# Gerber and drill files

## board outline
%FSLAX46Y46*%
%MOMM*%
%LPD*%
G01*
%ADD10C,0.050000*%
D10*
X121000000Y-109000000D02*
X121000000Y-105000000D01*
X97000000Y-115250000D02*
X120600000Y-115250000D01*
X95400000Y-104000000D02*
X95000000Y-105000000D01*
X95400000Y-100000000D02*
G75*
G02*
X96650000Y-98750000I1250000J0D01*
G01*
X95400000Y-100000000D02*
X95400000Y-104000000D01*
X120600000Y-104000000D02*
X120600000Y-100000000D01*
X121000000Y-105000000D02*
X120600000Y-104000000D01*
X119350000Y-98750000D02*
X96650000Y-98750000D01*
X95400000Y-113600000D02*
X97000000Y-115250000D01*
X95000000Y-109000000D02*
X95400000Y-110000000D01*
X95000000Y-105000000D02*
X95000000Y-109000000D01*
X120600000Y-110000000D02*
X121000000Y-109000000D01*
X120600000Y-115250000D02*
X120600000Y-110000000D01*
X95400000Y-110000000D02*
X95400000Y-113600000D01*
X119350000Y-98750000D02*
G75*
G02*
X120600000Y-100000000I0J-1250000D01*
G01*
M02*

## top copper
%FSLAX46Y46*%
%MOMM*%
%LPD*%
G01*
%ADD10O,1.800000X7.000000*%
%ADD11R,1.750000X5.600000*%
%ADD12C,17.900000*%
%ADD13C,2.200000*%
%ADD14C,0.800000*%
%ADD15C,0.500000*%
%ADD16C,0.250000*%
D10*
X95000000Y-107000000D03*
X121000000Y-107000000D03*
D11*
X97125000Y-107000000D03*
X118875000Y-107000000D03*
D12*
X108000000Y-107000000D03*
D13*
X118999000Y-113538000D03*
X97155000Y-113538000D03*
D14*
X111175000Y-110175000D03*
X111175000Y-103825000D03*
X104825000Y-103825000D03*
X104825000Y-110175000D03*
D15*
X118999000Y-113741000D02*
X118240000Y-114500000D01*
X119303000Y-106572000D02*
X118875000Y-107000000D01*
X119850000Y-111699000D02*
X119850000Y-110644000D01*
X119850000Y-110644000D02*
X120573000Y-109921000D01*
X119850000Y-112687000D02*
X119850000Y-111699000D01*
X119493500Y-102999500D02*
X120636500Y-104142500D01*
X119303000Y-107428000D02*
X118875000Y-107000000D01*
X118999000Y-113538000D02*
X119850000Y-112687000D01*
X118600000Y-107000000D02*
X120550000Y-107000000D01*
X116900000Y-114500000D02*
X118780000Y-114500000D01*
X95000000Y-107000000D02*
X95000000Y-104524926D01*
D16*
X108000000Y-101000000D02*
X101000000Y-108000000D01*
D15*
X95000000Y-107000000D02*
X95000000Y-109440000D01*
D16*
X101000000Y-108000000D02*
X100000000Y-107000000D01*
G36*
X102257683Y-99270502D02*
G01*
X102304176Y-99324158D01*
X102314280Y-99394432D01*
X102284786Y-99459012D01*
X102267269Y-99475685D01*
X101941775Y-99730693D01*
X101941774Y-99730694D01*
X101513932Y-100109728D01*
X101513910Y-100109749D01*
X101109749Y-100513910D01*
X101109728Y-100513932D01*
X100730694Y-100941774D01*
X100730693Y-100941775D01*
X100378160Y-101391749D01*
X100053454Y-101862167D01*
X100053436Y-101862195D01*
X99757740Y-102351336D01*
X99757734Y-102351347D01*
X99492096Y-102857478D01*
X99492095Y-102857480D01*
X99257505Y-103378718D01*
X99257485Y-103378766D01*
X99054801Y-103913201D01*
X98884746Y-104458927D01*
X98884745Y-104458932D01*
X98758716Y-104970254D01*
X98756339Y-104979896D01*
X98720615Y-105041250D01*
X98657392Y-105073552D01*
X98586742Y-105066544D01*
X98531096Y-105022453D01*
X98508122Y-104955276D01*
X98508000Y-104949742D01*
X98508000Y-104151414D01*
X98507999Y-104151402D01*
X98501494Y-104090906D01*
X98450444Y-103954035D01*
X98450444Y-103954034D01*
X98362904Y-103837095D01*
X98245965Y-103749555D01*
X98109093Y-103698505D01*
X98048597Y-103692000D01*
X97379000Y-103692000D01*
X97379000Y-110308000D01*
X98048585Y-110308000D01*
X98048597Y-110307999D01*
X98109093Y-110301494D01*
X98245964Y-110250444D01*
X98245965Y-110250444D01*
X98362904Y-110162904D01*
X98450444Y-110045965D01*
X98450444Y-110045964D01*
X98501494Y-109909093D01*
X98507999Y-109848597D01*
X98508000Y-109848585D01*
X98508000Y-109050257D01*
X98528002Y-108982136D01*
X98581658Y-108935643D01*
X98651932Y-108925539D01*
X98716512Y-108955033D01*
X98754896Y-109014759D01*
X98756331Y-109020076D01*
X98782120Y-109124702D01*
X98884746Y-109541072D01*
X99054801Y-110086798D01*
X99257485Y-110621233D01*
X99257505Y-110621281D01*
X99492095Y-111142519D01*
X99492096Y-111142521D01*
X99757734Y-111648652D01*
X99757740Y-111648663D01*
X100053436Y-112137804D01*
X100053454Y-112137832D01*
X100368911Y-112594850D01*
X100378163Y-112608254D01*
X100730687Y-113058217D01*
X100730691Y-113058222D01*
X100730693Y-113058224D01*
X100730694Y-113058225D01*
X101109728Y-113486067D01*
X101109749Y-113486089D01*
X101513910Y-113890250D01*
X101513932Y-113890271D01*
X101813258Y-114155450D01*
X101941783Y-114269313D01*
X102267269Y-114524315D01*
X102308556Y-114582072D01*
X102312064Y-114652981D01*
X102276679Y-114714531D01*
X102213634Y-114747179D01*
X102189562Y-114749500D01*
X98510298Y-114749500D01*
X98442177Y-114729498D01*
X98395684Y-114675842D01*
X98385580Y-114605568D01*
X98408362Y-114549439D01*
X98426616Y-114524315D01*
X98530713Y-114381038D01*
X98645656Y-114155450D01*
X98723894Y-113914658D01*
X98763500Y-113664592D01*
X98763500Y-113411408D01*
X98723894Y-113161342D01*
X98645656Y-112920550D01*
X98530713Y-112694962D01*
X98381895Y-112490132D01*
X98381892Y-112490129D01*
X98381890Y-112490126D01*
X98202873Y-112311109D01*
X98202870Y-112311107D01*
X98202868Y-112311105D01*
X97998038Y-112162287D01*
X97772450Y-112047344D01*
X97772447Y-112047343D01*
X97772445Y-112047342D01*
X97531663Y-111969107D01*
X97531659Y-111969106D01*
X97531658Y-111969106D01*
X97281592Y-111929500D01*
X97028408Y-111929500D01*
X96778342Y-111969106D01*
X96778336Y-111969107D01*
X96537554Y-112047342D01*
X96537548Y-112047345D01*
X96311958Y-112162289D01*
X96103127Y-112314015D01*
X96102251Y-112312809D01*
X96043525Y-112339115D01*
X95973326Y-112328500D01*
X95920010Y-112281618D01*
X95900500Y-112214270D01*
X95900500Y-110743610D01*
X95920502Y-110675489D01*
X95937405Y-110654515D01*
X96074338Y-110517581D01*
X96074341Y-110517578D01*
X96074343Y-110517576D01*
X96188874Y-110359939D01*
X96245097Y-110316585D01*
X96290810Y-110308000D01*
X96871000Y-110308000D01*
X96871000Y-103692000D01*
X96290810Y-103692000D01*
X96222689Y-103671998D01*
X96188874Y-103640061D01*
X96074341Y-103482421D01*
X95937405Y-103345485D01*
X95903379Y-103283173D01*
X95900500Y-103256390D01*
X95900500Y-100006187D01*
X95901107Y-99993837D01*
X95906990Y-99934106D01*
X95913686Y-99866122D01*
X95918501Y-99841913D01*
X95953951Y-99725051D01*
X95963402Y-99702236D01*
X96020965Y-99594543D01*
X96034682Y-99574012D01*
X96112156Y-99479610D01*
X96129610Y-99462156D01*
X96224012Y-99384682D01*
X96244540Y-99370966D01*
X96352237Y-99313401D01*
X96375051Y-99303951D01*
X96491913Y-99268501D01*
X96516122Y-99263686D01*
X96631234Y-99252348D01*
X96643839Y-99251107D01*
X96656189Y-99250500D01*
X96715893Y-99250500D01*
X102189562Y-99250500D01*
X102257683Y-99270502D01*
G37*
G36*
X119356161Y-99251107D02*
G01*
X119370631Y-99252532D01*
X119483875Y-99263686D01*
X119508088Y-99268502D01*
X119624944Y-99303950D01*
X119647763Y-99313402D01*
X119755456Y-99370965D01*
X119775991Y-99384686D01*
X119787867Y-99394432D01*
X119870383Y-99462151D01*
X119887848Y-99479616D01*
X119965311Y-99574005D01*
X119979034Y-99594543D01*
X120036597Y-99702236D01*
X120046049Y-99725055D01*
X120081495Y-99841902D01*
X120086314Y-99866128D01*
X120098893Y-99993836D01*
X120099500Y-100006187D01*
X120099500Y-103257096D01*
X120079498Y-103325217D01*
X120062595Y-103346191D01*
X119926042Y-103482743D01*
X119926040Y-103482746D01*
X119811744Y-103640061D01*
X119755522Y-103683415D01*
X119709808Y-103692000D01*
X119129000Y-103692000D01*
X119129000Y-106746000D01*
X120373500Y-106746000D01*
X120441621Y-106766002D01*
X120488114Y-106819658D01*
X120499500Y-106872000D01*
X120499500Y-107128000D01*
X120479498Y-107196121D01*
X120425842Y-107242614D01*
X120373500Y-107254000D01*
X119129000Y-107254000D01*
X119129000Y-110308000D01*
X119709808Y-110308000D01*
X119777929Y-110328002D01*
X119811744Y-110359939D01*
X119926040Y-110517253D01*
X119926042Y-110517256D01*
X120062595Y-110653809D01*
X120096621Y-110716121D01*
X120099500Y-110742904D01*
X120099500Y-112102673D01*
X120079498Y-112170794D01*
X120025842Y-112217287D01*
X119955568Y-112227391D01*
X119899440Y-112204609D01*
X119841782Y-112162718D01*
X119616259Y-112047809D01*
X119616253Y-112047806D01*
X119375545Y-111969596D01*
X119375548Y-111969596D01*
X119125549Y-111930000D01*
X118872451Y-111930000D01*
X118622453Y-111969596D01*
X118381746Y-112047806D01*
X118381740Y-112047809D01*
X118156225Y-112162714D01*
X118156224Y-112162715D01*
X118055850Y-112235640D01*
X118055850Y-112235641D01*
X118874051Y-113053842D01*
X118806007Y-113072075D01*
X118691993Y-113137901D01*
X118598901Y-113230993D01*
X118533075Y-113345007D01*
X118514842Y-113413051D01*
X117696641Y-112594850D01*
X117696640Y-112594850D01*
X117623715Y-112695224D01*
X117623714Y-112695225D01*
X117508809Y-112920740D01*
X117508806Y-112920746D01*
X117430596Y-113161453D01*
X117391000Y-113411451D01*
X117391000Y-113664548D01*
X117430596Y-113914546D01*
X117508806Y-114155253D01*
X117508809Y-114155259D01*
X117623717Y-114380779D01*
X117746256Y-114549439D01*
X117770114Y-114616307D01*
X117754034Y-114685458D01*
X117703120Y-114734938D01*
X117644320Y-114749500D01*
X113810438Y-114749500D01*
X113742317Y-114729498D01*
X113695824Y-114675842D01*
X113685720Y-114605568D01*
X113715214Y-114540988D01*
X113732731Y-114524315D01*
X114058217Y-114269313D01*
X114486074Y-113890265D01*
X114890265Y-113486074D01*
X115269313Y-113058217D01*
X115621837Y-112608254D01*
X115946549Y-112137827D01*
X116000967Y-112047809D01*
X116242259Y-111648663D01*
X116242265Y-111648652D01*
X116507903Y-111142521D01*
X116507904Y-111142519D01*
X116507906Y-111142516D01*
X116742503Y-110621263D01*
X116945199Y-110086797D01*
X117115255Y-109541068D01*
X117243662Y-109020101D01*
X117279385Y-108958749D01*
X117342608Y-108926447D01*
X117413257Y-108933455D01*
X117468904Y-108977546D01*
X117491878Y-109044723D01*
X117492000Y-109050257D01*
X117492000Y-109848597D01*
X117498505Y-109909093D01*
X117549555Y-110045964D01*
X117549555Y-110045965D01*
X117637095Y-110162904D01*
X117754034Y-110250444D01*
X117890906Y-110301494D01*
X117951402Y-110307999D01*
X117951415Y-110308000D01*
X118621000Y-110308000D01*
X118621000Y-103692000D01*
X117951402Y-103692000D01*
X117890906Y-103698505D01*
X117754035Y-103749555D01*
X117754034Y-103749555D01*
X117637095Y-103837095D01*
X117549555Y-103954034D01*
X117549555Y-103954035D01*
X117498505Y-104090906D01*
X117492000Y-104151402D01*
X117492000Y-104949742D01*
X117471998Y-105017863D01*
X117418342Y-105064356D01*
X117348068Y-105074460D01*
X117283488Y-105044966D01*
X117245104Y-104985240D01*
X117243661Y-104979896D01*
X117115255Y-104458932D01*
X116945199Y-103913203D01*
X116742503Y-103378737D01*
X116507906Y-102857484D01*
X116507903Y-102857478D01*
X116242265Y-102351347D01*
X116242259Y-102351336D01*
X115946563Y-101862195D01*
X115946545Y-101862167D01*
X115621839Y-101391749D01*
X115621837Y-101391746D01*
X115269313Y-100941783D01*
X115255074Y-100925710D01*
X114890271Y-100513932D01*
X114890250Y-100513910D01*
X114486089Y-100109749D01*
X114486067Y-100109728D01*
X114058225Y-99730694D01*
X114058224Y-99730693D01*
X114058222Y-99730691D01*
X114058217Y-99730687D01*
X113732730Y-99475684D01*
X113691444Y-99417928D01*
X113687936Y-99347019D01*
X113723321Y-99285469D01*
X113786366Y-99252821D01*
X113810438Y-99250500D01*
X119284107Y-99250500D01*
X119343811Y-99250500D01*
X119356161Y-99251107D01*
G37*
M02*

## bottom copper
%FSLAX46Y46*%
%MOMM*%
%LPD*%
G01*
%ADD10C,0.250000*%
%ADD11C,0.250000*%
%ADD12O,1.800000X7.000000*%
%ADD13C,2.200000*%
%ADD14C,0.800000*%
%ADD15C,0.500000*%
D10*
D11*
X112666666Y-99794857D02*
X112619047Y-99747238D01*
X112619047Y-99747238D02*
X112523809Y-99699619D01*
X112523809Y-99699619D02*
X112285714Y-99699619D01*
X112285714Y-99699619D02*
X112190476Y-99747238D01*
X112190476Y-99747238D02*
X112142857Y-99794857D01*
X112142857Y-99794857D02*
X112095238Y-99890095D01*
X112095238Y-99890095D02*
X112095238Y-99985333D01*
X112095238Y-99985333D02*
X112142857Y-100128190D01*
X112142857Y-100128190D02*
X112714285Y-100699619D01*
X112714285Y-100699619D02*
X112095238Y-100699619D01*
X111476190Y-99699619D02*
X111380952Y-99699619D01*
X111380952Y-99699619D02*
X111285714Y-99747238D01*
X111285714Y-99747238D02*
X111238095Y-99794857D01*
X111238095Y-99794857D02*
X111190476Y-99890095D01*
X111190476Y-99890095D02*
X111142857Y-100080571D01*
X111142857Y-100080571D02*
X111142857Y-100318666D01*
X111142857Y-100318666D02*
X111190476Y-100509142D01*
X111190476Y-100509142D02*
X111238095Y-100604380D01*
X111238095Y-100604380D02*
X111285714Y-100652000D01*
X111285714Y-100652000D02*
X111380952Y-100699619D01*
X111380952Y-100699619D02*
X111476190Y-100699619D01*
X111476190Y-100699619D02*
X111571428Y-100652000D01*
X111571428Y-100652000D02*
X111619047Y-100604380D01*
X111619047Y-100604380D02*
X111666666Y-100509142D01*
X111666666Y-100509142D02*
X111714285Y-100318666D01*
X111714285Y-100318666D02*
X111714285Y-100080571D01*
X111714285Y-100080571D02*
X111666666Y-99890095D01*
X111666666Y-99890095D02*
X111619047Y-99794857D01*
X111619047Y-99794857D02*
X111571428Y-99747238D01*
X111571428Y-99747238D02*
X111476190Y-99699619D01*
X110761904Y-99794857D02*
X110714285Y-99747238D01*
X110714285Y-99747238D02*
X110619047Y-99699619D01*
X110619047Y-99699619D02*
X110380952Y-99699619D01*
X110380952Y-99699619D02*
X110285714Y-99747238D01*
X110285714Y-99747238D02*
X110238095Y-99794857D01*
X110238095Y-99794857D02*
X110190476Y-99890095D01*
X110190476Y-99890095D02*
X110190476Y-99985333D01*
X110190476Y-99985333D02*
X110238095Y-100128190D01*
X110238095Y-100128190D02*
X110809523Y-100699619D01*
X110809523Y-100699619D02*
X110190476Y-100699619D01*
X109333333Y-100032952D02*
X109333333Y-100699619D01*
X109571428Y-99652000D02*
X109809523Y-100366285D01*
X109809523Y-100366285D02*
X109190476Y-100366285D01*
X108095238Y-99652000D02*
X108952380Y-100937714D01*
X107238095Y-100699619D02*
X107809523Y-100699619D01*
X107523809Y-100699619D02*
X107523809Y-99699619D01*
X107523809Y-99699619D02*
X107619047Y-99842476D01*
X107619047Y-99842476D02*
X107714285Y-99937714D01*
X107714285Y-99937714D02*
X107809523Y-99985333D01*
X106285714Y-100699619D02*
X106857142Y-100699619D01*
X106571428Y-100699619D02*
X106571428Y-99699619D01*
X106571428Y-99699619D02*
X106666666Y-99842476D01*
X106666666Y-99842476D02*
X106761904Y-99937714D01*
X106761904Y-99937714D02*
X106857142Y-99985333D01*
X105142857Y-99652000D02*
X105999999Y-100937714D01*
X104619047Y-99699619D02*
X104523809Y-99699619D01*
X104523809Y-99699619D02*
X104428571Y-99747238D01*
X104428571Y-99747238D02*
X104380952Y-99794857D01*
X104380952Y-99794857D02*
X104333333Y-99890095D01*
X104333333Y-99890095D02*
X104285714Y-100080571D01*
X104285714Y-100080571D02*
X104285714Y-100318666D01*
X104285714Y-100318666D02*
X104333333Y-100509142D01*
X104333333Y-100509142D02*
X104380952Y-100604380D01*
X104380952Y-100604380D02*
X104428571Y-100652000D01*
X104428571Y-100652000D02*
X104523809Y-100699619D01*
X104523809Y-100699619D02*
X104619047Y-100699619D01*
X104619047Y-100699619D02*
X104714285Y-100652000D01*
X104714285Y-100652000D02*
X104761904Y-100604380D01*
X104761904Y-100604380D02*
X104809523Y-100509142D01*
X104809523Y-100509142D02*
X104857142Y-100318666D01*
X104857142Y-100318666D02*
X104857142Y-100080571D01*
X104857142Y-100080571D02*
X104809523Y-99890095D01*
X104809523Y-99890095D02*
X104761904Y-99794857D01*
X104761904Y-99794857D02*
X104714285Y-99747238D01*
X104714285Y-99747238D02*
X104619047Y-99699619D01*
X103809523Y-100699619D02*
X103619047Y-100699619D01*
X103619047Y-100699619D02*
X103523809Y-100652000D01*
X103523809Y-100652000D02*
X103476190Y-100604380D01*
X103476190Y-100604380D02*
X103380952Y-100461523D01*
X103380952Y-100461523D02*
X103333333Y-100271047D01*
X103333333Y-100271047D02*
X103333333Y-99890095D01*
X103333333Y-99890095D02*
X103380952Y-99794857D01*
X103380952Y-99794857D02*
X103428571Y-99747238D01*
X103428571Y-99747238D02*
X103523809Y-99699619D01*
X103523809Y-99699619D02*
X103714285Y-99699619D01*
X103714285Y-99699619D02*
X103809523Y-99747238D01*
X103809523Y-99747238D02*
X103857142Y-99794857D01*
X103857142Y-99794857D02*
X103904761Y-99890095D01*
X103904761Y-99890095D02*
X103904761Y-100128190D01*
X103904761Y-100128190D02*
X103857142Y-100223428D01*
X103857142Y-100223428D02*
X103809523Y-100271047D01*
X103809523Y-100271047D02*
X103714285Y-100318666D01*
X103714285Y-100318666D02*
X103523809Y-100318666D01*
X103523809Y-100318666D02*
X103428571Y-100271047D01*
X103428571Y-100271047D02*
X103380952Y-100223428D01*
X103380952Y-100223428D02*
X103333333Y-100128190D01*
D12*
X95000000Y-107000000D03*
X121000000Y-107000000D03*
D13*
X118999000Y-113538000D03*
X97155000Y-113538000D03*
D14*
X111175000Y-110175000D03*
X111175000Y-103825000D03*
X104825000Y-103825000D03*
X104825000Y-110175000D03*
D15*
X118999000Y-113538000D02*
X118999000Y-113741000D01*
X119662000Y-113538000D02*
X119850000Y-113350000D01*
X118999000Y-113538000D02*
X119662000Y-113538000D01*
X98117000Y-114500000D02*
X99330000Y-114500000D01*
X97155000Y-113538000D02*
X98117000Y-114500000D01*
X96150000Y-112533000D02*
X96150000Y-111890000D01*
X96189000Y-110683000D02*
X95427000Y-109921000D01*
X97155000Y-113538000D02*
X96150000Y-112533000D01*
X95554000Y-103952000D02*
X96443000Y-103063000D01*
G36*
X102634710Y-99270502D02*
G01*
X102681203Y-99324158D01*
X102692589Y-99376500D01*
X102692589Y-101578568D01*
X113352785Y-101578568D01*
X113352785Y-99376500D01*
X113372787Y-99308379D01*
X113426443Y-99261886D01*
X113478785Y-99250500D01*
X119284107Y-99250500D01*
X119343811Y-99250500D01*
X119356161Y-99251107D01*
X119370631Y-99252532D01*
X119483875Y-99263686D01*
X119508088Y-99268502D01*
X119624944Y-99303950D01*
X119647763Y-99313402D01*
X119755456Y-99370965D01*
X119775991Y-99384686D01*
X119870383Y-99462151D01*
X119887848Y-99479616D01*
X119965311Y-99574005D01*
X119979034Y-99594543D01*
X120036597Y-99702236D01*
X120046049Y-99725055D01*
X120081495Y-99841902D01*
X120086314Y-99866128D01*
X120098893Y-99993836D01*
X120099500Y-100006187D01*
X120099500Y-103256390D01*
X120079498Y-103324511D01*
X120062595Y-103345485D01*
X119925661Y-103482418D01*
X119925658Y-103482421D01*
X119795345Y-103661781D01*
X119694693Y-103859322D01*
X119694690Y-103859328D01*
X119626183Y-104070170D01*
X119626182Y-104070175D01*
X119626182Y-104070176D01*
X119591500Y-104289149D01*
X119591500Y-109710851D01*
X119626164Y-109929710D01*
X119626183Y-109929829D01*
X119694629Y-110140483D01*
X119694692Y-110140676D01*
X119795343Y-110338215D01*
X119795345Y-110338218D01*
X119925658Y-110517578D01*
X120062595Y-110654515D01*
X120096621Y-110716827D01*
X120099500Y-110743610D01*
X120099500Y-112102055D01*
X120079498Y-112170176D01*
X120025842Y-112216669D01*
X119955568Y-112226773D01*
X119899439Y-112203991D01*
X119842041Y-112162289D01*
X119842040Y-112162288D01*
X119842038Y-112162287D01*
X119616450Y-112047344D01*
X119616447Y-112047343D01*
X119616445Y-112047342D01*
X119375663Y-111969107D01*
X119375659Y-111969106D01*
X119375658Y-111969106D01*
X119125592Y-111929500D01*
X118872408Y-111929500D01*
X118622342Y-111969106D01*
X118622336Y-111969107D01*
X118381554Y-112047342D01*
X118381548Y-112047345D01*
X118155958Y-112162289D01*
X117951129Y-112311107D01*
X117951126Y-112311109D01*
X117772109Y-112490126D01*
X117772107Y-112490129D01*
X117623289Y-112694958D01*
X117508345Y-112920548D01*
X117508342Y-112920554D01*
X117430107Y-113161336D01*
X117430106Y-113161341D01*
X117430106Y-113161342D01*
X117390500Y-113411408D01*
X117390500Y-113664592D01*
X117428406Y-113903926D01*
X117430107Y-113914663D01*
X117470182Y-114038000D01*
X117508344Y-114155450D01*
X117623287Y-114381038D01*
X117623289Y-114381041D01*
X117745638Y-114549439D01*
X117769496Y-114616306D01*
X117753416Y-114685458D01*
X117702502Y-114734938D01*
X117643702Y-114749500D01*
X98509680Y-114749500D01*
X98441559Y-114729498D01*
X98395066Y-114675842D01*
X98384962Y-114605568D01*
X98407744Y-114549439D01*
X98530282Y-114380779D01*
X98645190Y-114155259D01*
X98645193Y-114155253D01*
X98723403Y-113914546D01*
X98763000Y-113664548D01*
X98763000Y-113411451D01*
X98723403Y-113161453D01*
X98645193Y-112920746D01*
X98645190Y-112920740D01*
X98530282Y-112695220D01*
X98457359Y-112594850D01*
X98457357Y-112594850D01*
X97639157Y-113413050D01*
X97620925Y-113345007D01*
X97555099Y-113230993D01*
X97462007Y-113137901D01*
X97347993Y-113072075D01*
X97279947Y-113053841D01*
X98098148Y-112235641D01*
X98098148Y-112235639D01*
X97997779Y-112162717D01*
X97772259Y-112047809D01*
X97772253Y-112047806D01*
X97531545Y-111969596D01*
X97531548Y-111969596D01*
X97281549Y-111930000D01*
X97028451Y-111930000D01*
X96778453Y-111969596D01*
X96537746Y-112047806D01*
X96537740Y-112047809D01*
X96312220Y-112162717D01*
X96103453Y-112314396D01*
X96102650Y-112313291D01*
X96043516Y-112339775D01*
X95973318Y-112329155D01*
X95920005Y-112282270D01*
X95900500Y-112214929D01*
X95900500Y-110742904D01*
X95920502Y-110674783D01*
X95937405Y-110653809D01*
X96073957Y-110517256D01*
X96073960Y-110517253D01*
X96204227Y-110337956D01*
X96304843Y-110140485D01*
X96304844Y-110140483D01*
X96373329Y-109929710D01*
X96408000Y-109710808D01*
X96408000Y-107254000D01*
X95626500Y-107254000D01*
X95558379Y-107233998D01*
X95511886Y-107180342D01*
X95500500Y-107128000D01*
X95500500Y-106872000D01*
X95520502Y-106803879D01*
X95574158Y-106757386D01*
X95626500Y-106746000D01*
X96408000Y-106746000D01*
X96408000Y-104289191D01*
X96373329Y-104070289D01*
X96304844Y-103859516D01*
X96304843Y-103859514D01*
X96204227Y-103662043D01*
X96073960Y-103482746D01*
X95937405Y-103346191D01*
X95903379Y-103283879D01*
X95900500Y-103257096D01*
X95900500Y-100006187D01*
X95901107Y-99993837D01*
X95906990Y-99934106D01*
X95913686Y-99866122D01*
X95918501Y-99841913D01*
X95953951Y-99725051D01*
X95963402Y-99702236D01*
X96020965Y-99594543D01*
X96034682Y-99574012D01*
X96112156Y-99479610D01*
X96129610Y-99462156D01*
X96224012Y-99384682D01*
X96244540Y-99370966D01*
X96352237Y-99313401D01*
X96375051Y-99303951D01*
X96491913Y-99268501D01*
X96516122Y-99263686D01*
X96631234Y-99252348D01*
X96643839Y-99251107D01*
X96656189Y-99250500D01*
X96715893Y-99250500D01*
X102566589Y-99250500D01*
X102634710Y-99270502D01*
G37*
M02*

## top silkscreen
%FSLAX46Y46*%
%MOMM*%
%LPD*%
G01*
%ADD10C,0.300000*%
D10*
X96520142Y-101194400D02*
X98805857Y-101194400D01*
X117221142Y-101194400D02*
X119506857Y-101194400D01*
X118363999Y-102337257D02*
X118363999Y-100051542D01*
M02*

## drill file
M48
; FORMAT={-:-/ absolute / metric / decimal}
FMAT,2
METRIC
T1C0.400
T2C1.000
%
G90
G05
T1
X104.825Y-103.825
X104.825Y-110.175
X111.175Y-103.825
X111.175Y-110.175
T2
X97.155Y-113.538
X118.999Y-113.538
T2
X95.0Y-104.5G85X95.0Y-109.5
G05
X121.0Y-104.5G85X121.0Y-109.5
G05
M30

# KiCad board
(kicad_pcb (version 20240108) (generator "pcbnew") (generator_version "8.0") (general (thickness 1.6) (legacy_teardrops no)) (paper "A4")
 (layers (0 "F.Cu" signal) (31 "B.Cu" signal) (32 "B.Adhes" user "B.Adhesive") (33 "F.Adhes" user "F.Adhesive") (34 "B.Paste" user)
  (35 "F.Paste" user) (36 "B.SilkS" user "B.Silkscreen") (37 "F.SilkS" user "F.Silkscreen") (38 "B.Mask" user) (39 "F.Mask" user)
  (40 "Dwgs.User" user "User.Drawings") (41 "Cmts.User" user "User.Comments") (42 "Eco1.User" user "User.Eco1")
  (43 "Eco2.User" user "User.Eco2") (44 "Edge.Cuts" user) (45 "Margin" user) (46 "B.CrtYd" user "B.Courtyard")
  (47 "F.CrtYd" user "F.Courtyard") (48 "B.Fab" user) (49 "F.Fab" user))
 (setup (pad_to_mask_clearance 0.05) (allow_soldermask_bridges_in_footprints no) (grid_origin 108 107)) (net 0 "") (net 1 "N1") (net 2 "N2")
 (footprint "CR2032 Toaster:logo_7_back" (layer "F.Cu") (at 114 106.25)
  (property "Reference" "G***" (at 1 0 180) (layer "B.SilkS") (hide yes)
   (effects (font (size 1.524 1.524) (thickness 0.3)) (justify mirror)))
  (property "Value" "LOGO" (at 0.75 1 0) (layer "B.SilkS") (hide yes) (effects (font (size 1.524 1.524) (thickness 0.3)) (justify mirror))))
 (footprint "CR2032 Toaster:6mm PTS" (layer "F.Cu") (at 95 107)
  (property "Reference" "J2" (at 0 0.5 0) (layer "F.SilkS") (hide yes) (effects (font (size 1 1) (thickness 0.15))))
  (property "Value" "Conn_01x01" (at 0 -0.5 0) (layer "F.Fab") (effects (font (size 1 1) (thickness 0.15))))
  (pad "1" thru_hole oval (at 0 0) (size 1.8 7) (drill oval 1 6) (layers "*.Cu" "*.Mask") (remove_unused_layers no) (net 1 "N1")))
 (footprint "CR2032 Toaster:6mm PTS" (layer "F.Cu") (at 121 107)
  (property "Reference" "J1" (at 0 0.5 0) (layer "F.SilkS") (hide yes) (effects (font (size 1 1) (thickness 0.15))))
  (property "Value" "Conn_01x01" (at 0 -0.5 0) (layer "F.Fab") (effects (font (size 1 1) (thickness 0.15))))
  (pad "1" thru_hole oval (at 0 0) (size 1.8 7) (drill oval 1 6) (layers "*.Cu" "*.Mask") (remove_unused_layers no) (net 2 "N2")))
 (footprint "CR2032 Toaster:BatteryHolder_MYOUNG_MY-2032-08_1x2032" (layer "F.Cu") (at 108 107)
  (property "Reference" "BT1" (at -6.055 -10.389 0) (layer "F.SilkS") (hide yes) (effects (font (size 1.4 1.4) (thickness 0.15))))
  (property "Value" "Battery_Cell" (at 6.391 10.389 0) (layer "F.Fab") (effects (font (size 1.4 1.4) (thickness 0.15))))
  (pad "1" smd rect (at -10.875 0) (size 1.75 5.6) (layers "F.Cu" "F.Paste" "F.Mask") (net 2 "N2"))
  (pad "1" smd rect (at 10.875 0) (size 1.75 5.6) (layers "F.Cu" "F.Paste" "F.Mask") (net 2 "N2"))
  (pad "2" smd circle (at 0 0) (size 17.9 17.9) (layers "F.Cu" "F.Mask") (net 1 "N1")))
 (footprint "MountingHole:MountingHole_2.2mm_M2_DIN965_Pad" (layer "F.Cu") (at 118.999 113.538)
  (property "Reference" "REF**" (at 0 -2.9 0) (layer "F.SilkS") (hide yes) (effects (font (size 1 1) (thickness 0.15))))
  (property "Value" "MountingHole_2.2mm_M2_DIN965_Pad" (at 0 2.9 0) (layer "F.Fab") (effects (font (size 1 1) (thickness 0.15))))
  (pad "1" thru_hole circle (at 0 0) (size 2.2 2.2) (drill 1) (layers "*.Cu" "*.Mask") (remove_unused_layers no) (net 2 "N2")))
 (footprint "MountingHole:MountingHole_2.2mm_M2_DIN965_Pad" (layer "F.Cu") (at 97.155 113.538)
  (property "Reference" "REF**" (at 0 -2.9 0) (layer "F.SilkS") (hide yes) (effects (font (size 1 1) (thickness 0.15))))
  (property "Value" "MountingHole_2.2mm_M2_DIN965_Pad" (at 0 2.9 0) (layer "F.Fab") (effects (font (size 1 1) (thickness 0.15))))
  (pad "1" thru_hole circle (at 0 0) (size 2.2 2.2) (drill 1) (layers "*.Cu" "*.Mask") (remove_unused_layers no) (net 1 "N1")))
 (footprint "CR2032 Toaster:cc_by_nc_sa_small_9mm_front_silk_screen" (layer "B.Cu") (at 107.95 113.5 180)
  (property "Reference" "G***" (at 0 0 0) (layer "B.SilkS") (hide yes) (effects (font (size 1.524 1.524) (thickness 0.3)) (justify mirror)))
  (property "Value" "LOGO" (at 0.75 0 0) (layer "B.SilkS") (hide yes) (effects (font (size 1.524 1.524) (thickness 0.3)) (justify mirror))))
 (gr_line (start 121 109) (end 121 105) (stroke (width 0.05) (type solid)) (layer "Edge.Cuts"))
 (gr_line (start 97 115.25) (end 120.6 115.25) (stroke (width 0.05) (type solid)) (layer "Edge.Cuts"))
 (gr_line (start 95.4 104) (end 95 105) (stroke (width 0.05) (type solid)) (layer "Edge.Cuts"))
 (gr_arc (start 95.4 100) (mid 95.766117 99.116117) (end 96.65 98.75) (stroke (width 0.05) (type solid)) (layer "Edge.Cuts"))
 (gr_line (start 95.4 100) (end 95.4 104) (stroke (width 0.05) (type solid)) (layer "Edge.Cuts"))
 (gr_line (start 120.6 104) (end 120.6 100) (stroke (width 0.05) (type solid)) (layer "Edge.Cuts"))
 (gr_line (start 121 105) (end 120.6 104) (stroke (width 0.05) (type solid)) (layer "Edge.Cuts"))
 (gr_line (start 119.35 98.75) (end 96.65 98.75) (stroke (width 0.05) (type solid)) (layer "Edge.Cuts"))
 (gr_line (start 95.4 113.6) (end 97 115.25) (stroke (width 0.05) (type solid)) (layer "Edge.Cuts"))
 (gr_line (start 95 109) (end 95.4 110) (stroke (width 0.05) (type solid)) (layer "Edge.Cuts"))
 (gr_line (start 95 105) (end 95 109) (stroke (width 0.05) (type solid)) (layer "Edge.Cuts"))
 (gr_line (start 120.6 110) (end 121 109) (stroke (width 0.05) (type solid)) (layer "Edge.Cuts"))
 (gr_line (start 120.6 115.25) (end 120.6 110) (stroke (width 0.05) (type solid)) (layer "Edge.Cuts"))
 (gr_line (start 95.4 110) (end 95.4 113.6) (stroke (width 0.05) (type solid)) (layer "Edge.Cuts"))
 (gr_arc (start 119.35 98.75) (mid 120.233883 99.116117) (end 120.6 100) (stroke (width 0.05) (type solid)) (layer "Edge.Cuts"))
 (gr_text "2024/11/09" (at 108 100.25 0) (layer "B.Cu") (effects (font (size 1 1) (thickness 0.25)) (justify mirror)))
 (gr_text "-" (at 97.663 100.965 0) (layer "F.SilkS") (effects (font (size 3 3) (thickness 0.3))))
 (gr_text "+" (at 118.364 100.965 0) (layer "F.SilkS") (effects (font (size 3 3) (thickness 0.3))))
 (segment (start 118.999 113.741) (end 118.24 114.5) (width 0.5) (layer "F.Cu") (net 2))
 (segment (start 119.303 106.572) (end 118.875 107) (width 0.5) (layer "F.Cu") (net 2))
 (segment (start 119.85 111.699) (end 119.85 110.644) (width 0.5) (layer "F.Cu") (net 2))
 (segment (start 119.85 110.644) (end 120.573 109.921) (width 0.5) (layer "F.Cu") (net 2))
 (segment (start 119.85 112.687) (end 119.85 111.699) (width 0.5) (layer "F.Cu") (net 2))
 (segment (start 119.4935 102.9995) (end 120.6365 104.1425) (width 0.5) (layer "F.Cu") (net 2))
 (segment (start 119.303 107.428) (end 118.875 107) (width 0.5) (layer "F.Cu") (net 2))
 (segment (start 118.999 113.538) (end 119.85 112.687) (width 0.5) (layer "F.Cu") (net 2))
 (segment (start 118.6 107) (end 120.55 107) (width 0.5) (layer "F.Cu") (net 2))
 (segment (start 116.9 114.5) (end 118.78 114.5) (width 0.5) (layer "F.Cu") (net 2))
 (segment (start 118.999 113.538) (end 118.999 113.741) (width 0.5) (layer "B.Cu") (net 2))
 (segment (start 119.662 113.538) (end 119.85 113.35) (width 0.5) (layer "B.Cu") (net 2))
 (segment (start 118.999 113.538) (end 119.662 113.538) (width 0.5) (layer "B.Cu") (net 2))
 (segment (start 95 107) (end 95 104.524926) (width 0.5) (layer "F.Cu") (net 1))
 (segment (start 108 101) (end 101 108) (width 0.25) (layer "F.Cu") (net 1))
 (segment (start 95 107) (end 95 109.44) (width 0.5) (layer "F.Cu") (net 1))
 (segment (start 101 108) (end 100 107) (width 0.25) (layer "F.Cu") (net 1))
 (via (at 111.175 110.175) (size 0.8) (drill 0.4) (layers "F.Cu" "B.Cu") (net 1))
 (via (at 111.175 103.825) (size 0.8) (drill 0.4) (layers "F.Cu" "B.Cu") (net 1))
 (via (at 104.825 103.825) (size 0.8) (drill 0.4) (layers "F.Cu" "B.Cu") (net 1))
 (via (at 104.825 110.175) (size 0.8) (drill 0.4) (layers "F.Cu" "B.Cu") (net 1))
 (segment (start 98.117 114.5) (end 99.33 114.5) (width 0.5) (layer "B.Cu") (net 1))
 (segment (start 97.155 113.538) (end 98.117 114.5) (width 0.5) (layer "B.Cu") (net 1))
 (segment (start 96.15 112.533) (end 96.15 111.89) (width 0.5) (layer "B.Cu") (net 1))
 (segment (start 96.189 110.683) (end 95.427 109.921) (width 0.5) (layer "B.Cu") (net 1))
 (segment (start 97.155 113.538) (end 96.15 112.533) (width 0.5) (layer "B.Cu") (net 1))
 (segment (start 95.554 103.952) (end 96.443 103.063) (width 0.5) (layer "B.Cu") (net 1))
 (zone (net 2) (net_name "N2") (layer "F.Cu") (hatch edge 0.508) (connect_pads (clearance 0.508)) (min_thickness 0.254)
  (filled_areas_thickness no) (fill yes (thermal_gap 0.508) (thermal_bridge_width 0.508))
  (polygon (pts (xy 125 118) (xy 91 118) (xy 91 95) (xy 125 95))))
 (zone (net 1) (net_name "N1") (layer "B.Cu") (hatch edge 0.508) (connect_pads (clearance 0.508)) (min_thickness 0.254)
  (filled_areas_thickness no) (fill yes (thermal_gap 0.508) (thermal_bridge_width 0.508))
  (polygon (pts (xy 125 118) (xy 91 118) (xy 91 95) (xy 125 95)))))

